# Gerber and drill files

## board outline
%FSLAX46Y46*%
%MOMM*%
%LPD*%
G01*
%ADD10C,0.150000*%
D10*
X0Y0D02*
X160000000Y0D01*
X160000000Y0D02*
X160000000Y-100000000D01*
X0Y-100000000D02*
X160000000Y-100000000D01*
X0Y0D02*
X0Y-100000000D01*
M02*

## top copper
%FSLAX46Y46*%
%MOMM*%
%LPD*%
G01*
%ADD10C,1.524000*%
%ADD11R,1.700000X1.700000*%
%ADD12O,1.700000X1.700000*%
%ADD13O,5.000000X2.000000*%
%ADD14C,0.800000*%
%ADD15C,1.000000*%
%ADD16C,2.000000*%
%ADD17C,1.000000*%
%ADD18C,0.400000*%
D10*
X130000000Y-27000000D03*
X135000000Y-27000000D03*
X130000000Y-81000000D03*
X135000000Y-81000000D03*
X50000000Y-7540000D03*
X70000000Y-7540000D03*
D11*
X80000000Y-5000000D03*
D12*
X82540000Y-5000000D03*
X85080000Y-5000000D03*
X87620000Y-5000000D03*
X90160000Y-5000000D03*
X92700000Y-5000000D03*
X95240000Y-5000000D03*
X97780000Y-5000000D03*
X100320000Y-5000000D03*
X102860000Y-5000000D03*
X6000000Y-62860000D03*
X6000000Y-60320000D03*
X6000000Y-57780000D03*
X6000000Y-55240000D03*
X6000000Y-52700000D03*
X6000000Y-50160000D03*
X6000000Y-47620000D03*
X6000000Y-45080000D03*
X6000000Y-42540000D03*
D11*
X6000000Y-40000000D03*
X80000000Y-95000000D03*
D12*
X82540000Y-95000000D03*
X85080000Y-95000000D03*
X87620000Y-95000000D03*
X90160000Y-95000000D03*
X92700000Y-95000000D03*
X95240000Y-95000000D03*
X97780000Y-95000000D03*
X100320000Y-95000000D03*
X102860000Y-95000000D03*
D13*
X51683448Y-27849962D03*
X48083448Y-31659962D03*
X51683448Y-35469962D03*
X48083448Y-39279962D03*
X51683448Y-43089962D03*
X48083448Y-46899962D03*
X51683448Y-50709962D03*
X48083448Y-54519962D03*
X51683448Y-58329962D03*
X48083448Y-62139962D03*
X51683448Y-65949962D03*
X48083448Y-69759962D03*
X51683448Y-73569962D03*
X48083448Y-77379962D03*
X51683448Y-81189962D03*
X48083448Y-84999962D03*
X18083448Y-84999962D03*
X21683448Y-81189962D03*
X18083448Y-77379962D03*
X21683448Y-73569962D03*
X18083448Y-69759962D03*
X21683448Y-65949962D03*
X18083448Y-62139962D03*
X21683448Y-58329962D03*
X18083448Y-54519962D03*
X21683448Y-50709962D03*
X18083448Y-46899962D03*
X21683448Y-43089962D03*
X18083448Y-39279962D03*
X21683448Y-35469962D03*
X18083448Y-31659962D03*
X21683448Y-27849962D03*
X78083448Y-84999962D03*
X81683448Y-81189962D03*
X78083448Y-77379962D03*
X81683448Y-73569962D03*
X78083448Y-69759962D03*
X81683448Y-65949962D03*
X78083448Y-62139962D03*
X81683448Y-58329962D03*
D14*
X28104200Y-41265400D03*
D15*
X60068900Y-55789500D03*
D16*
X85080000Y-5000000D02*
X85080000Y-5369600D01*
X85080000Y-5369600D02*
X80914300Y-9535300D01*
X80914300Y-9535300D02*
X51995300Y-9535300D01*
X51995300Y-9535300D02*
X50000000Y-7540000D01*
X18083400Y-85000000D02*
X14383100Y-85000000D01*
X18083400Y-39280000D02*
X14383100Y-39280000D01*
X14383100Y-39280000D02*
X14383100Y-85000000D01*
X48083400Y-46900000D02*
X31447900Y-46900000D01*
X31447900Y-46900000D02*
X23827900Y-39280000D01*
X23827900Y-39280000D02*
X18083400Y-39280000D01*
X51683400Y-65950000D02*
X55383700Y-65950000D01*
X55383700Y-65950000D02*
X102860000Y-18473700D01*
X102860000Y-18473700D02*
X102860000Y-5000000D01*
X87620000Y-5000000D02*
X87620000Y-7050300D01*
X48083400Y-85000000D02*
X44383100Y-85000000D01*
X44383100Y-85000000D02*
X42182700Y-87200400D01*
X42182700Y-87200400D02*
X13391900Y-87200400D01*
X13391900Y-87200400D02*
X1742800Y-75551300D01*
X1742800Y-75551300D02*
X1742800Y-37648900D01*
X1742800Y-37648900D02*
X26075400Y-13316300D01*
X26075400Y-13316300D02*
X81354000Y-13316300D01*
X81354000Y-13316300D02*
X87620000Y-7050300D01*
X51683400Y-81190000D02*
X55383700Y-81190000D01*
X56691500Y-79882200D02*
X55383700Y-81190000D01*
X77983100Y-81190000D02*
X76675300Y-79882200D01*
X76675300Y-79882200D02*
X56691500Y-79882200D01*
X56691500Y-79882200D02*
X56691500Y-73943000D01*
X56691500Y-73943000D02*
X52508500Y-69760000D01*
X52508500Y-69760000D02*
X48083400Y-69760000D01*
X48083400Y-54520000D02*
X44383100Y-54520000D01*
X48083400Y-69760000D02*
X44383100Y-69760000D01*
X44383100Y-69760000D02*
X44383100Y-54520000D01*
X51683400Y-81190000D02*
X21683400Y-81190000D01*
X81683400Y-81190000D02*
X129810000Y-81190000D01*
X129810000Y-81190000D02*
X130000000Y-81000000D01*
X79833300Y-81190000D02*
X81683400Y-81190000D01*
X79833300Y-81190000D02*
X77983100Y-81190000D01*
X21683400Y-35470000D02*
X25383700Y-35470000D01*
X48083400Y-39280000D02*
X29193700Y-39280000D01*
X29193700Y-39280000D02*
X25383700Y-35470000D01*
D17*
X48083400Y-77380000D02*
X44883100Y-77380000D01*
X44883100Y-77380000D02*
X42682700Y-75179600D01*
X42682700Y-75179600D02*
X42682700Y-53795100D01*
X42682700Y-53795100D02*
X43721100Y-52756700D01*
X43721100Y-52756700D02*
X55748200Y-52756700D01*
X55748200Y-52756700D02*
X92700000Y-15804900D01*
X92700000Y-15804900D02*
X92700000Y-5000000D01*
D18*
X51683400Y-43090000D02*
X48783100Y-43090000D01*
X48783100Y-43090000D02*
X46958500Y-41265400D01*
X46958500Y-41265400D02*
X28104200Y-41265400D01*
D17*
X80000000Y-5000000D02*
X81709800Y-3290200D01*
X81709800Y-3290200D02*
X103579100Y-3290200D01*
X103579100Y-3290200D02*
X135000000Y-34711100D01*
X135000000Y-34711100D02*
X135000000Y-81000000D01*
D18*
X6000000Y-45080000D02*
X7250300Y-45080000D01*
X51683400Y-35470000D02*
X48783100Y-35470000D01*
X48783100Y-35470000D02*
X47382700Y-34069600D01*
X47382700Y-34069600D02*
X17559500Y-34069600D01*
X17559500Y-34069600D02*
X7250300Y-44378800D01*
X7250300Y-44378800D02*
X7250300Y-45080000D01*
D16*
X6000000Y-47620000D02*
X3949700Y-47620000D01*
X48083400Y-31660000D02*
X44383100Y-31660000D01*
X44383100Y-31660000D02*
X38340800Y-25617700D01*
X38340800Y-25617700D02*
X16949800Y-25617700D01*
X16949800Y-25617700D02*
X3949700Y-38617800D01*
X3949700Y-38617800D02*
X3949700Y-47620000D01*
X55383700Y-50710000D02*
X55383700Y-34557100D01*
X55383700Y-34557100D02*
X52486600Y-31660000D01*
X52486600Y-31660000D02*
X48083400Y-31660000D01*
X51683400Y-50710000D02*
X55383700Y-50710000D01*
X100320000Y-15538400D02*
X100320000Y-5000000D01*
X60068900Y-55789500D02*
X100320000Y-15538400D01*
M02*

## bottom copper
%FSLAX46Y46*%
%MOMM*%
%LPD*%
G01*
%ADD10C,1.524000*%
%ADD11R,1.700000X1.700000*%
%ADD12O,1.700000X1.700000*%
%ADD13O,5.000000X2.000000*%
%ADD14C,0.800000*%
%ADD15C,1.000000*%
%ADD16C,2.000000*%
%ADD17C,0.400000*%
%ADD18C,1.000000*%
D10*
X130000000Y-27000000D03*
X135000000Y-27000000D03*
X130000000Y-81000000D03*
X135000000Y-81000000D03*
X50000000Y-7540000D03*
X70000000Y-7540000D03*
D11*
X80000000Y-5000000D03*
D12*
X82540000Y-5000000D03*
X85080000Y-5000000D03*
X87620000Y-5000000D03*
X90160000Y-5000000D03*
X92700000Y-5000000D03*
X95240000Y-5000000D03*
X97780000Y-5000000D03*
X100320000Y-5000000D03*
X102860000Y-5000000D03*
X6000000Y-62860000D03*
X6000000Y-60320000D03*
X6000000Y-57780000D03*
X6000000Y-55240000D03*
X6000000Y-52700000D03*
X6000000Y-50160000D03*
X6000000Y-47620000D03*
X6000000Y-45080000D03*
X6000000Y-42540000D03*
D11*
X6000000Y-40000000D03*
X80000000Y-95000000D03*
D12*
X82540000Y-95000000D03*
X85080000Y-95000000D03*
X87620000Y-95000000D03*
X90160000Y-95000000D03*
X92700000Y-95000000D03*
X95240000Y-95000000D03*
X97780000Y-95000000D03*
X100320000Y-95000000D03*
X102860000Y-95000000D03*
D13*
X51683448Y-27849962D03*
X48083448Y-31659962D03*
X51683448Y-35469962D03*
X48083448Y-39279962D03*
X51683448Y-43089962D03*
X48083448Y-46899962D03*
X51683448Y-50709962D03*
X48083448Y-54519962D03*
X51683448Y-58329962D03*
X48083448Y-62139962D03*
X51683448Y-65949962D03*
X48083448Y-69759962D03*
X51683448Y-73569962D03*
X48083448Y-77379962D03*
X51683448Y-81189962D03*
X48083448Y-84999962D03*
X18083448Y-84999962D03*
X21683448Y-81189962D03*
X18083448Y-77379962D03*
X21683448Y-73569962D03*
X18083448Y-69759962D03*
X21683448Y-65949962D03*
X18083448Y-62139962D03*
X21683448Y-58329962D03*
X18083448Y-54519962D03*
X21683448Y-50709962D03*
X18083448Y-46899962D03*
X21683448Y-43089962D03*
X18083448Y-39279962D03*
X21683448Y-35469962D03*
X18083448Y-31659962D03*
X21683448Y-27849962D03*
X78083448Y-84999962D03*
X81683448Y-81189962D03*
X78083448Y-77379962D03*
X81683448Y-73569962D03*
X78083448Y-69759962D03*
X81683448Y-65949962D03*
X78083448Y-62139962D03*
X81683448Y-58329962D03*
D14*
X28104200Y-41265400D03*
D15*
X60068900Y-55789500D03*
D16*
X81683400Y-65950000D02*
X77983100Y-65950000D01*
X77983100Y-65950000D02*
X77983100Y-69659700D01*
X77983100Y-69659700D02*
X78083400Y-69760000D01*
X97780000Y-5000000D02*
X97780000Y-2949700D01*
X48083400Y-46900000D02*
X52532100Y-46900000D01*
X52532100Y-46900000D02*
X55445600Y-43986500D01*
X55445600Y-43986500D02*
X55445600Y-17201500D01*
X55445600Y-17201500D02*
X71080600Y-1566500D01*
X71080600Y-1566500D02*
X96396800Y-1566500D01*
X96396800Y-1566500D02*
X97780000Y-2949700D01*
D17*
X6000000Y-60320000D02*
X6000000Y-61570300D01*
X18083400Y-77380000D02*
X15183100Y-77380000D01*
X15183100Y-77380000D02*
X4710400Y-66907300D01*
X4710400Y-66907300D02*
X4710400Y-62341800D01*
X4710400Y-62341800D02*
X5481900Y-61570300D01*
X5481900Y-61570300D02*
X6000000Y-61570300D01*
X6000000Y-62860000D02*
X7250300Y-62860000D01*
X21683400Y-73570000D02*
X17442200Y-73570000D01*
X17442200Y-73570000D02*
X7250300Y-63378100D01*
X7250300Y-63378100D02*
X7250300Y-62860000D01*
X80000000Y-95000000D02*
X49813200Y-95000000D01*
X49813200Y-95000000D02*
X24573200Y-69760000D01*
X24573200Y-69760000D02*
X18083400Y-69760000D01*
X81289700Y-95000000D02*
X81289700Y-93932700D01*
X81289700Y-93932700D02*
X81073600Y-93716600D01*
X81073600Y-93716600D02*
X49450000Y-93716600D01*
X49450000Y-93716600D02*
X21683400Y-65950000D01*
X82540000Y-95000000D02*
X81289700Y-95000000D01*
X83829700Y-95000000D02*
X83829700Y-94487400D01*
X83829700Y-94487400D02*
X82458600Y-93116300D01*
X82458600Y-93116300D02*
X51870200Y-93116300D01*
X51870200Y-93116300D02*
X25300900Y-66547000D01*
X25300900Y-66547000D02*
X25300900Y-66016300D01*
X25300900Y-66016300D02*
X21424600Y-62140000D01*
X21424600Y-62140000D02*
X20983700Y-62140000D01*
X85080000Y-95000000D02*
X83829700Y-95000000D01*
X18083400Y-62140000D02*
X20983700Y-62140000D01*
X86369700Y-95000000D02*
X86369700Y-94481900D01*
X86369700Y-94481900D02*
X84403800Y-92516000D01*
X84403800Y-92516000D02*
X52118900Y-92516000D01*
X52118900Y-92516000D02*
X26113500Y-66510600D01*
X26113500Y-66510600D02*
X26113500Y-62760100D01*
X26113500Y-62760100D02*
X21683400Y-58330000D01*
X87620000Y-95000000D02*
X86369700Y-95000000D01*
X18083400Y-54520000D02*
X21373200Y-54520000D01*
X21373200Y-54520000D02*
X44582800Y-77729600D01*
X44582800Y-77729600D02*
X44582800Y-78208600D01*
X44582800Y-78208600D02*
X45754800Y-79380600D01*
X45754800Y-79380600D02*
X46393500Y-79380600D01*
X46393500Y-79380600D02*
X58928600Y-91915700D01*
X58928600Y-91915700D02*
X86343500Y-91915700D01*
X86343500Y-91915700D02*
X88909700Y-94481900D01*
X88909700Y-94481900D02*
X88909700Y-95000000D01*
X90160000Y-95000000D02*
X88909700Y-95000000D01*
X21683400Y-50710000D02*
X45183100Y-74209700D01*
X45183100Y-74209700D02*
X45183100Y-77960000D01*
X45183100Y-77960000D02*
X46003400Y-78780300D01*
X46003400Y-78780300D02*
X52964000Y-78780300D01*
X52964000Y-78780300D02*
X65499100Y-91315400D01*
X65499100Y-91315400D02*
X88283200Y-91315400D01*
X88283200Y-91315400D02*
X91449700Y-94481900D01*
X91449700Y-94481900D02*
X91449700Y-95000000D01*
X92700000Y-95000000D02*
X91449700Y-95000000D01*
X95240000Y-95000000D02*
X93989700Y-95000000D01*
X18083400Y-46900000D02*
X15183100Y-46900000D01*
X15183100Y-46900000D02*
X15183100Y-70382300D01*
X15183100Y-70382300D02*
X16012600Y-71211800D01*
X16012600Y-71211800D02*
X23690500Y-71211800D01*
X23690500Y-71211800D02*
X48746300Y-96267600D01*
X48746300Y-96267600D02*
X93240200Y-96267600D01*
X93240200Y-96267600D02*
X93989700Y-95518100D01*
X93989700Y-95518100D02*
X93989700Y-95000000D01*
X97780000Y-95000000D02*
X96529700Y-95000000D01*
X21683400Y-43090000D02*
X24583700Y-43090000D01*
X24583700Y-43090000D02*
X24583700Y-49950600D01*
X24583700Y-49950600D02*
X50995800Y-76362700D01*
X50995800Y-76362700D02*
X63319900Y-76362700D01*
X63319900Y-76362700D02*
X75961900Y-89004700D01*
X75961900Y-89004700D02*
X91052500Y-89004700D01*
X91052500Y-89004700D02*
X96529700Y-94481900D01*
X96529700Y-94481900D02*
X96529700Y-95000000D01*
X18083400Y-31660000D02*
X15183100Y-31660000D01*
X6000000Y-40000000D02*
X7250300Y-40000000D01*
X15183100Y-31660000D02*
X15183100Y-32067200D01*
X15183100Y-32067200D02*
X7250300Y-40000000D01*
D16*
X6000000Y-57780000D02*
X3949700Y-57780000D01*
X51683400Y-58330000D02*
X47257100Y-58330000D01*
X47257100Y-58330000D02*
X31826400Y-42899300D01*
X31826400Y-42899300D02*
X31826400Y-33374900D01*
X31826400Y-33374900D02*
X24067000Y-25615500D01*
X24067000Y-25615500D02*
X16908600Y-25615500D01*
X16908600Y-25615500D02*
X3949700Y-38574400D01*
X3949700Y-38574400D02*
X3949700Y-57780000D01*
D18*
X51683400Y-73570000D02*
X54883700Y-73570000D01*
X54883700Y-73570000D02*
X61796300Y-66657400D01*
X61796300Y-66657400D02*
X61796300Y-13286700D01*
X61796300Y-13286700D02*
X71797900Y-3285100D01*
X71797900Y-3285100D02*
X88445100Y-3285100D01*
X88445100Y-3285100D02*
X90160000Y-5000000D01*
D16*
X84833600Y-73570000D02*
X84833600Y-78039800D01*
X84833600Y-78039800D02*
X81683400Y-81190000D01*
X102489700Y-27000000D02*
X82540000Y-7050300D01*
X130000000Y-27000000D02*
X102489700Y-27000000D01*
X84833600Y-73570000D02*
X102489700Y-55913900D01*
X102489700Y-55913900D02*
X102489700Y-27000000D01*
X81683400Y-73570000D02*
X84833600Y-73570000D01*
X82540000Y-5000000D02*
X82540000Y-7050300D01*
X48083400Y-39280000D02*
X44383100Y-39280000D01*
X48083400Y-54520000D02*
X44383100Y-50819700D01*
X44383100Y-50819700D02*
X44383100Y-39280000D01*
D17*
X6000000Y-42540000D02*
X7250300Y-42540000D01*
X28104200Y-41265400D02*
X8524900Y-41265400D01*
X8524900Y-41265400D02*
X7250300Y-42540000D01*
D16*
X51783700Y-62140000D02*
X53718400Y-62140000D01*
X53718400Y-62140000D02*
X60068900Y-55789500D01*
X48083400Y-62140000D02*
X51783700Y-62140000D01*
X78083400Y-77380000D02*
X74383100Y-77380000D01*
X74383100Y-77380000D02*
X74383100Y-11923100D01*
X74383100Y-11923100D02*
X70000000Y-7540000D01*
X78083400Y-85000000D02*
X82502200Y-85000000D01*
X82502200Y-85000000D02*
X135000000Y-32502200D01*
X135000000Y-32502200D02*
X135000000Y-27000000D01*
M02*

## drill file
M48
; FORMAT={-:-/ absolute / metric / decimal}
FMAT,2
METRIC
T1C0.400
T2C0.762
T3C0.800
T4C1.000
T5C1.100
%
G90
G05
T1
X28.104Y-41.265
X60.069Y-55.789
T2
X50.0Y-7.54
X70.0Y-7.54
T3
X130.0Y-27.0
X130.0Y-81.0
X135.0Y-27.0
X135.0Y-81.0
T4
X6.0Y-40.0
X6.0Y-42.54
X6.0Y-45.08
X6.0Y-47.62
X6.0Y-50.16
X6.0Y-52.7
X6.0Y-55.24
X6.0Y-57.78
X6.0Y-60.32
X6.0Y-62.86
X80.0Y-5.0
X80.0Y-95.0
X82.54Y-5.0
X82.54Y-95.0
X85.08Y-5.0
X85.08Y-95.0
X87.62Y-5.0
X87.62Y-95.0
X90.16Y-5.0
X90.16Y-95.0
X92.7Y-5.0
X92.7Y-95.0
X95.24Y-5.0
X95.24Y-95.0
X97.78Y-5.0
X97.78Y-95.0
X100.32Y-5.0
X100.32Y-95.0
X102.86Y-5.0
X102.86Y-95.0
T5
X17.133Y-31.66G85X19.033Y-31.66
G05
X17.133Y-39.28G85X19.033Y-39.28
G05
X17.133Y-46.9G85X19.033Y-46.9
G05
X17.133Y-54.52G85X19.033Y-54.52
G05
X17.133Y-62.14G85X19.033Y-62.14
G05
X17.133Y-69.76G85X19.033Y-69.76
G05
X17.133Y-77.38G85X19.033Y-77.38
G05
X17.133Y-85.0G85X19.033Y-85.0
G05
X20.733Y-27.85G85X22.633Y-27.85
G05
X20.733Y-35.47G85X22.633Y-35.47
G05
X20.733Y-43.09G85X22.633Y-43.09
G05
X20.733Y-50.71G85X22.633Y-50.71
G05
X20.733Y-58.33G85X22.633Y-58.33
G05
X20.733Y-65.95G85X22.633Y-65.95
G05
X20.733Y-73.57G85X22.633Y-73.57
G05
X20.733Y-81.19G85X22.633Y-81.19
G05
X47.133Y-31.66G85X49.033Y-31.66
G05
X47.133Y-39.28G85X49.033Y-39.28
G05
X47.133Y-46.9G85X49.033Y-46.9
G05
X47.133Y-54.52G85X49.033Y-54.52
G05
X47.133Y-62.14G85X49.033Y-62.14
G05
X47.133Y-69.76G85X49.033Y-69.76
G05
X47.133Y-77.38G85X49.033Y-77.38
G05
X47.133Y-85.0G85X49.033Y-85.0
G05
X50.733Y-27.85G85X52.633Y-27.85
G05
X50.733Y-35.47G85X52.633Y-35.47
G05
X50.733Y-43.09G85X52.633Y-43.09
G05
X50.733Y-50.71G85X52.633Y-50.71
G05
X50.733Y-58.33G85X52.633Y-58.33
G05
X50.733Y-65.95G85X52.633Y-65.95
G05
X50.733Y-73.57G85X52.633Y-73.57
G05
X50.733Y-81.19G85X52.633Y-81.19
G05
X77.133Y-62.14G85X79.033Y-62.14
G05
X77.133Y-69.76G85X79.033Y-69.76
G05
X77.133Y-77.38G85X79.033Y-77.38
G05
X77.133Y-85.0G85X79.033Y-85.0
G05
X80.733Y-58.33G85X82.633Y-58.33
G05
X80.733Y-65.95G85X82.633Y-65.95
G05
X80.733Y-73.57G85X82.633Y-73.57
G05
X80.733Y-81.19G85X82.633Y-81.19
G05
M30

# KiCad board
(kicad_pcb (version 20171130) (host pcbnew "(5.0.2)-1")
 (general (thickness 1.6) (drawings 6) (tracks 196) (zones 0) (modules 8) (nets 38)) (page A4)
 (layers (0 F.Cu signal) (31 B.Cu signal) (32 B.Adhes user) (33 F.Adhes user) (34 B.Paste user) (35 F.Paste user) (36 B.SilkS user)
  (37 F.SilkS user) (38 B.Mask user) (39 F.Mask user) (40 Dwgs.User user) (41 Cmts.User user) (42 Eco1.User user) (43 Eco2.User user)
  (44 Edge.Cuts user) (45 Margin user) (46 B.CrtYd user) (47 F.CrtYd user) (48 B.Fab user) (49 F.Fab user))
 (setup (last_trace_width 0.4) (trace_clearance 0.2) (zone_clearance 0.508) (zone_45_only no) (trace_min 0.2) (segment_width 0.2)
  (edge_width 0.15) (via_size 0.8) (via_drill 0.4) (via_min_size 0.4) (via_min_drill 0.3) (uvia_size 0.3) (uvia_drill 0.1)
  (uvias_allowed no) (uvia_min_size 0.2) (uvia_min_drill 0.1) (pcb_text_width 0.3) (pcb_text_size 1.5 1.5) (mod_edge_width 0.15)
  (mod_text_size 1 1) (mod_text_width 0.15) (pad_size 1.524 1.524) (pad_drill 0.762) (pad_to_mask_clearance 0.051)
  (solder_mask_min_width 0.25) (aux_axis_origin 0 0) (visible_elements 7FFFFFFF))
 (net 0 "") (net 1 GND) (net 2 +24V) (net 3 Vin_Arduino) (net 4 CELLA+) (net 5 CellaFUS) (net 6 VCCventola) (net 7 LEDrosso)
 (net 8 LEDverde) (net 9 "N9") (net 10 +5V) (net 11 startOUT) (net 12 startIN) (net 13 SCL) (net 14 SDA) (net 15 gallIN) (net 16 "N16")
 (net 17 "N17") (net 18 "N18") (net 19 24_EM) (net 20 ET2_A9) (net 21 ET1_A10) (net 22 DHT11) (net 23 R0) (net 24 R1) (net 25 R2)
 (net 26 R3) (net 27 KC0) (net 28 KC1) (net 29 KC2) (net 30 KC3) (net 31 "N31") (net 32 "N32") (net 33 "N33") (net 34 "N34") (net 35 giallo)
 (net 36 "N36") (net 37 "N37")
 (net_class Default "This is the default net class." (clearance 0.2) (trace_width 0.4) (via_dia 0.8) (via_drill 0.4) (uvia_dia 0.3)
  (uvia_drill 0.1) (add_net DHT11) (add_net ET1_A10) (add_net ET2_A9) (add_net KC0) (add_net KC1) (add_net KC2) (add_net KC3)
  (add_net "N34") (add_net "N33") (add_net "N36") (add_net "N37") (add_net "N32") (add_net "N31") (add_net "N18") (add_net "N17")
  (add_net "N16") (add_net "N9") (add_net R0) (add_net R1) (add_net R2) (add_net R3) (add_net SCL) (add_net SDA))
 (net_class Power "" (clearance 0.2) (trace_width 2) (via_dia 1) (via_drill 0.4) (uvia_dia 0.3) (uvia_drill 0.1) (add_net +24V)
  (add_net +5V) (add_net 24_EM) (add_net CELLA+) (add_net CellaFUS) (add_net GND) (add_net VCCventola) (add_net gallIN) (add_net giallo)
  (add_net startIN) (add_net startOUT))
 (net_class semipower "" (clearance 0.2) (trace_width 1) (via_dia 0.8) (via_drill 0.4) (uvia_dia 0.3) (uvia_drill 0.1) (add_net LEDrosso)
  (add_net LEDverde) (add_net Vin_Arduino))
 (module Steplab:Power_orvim (layer F.Cu) (at 130 23)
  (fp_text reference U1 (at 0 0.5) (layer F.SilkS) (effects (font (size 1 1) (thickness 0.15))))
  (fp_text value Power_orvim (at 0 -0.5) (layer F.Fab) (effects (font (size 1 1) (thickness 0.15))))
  (pad 2 thru_hole circle (at 0 4) (size 1.524 1.524) (drill 0.8) (layers *.Cu *.Mask) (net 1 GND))
  (pad 1 thru_hole circle (at 5 4) (size 1.524 1.524) (drill 0.8) (layers *.Cu *.Mask) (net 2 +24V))
  (pad 4 thru_hole circle (at 0 58) (size 1.524 1.524) (drill 0.8) (layers *.Cu *.Mask) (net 1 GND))
  (pad 3 thru_hole circle (at 5 58) (size 1.524 1.524) (drill 0.8) (layers *.Cu *.Mask) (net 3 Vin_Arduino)))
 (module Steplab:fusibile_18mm (layer F.Cu) (at 51.95 5)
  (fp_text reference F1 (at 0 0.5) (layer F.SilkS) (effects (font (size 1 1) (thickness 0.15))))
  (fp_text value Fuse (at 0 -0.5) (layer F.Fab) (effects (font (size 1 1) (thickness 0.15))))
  (pad 1 thru_hole circle (at -1.95 2.54) (size 1.524 1.524) (drill 0.762) (layers *.Cu *.Mask) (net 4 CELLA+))
  (pad 2 thru_hole circle (at 18.05 2.54) (size 1.524 1.524) (drill 0.762) (layers *.Cu *.Mask) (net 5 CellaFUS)))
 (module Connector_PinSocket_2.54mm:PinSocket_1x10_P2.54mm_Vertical (layer F.Cu) (at 80 5 90)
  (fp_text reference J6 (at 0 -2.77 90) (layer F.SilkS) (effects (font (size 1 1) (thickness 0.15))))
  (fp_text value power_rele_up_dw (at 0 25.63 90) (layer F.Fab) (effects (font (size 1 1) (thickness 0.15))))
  (pad 1 thru_hole rect (at 0 0 90) (size 1.7 1.7) (drill 1) (layers *.Cu *.Mask) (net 3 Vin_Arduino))
  (pad 2 thru_hole oval (at 0 2.54 90) (size 1.7 1.7) (drill 1) (layers *.Cu *.Mask) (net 1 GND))
  (pad 3 thru_hole oval (at 0 5.08 90) (size 1.7 1.7) (drill 1) (layers *.Cu *.Mask) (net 4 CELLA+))
  (pad 4 thru_hole oval (at 0 7.62 90) (size 1.7 1.7) (drill 1) (layers *.Cu *.Mask) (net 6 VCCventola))
  (pad 5 thru_hole oval (at 0 10.16 90) (size 1.7 1.7) (drill 1) (layers *.Cu *.Mask) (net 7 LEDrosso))
  (pad 6 thru_hole oval (at 0 12.7 90) (size 1.7 1.7) (drill 1) (layers *.Cu *.Mask) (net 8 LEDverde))
  (pad 7 thru_hole oval (at 0 15.24 90) (size 1.7 1.7) (drill 1) (layers *.Cu *.Mask) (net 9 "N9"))
  (pad 8 thru_hole oval (at 0 17.78 90) (size 1.7 1.7) (drill 1) (layers *.Cu *.Mask) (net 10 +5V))
  (pad 9 thru_hole oval (at 0 20.32 90) (size 1.7 1.7) (drill 1) (layers *.Cu *.Mask) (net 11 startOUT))
  (pad 10 thru_hole oval (at 0 22.86 90) (size 1.7 1.7) (drill 1) (layers *.Cu *.Mask) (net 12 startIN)))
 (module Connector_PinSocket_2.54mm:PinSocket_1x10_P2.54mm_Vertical (layer F.Cu) (at 6 40)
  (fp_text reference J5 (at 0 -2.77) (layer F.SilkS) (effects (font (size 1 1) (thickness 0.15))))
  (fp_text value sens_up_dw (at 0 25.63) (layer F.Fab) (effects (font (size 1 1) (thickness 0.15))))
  (pad 10 thru_hole oval (at 0 22.86) (size 1.7 1.7) (drill 1) (layers *.Cu *.Mask) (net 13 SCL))
  (pad 9 thru_hole oval (at 0 20.32) (size 1.7 1.7) (drill 1) (layers *.Cu *.Mask) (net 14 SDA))
  (pad 8 thru_hole oval (at 0 17.78) (size 1.7 1.7) (drill 1) (layers *.Cu *.Mask) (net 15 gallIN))
  (pad 7 thru_hole oval (at 0 15.24) (size 1.7 1.7) (drill 1) (layers *.Cu *.Mask) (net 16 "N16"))
  (pad 6 thru_hole oval (at 0 12.7) (size 1.7 1.7) (drill 1) (layers *.Cu *.Mask) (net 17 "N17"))
  (pad 5 thru_hole oval (at 0 10.16) (size 1.7 1.7) (drill 1) (layers *.Cu *.Mask) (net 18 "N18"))
  (pad 4 thru_hole oval (at 0 7.62) (size 1.7 1.7) (drill 1) (layers *.Cu *.Mask) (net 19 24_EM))
  (pad 3 thru_hole oval (at 0 5.08) (size 1.7 1.7) (drill 1) (layers *.Cu *.Mask) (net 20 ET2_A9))
  (pad 2 thru_hole oval (at 0 2.54) (size 1.7 1.7) (drill 1) (layers *.Cu *.Mask) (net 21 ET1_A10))
  (pad 1 thru_hole rect (at 0 0) (size 1.7 1.7) (drill 1) (layers *.Cu *.Mask) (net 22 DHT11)))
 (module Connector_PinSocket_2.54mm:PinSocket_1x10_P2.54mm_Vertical (layer F.Cu) (at 80 95 90)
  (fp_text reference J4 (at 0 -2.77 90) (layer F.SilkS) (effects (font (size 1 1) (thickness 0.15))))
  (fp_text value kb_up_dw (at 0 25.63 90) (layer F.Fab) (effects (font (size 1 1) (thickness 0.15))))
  (pad 1 thru_hole rect (at 0 0 90) (size 1.7 1.7) (drill 1) (layers *.Cu *.Mask) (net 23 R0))
  (pad 2 thru_hole oval (at 0 2.54 90) (size 1.7 1.7) (drill 1) (layers *.Cu *.Mask) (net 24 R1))
  (pad 3 thru_hole oval (at 0 5.08 90) (size 1.7 1.7) (drill 1) (layers *.Cu *.Mask) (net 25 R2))
  (pad 4 thru_hole oval (at 0 7.62 90) (size 1.7 1.7) (drill 1) (layers *.Cu *.Mask) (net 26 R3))
  (pad 5 thru_hole oval (at 0 10.16 90) (size 1.7 1.7) (drill 1) (layers *.Cu *.Mask) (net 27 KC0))
  (pad 6 thru_hole oval (at 0 12.7 90) (size 1.7 1.7) (drill 1) (layers *.Cu *.Mask) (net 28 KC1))
  (pad 7 thru_hole oval (at 0 15.24 90) (size 1.7 1.7) (drill 1) (layers *.Cu *.Mask) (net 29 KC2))
  (pad 8 thru_hole oval (at 0 17.78 90) (size 1.7 1.7) (drill 1) (layers *.Cu *.Mask) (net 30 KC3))
  (pad 9 thru_hole oval (at 0 20.32 90) (size 1.7 1.7) (drill 1) (layers *.Cu *.Mask) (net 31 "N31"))
  (pad 10 thru_hole oval (at 0 22.86 90) (size 1.7 1.7) (drill 1) (layers *.Cu *.Mask) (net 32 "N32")))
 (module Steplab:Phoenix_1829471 (layer F.Cu) (at 52 68.5137 180)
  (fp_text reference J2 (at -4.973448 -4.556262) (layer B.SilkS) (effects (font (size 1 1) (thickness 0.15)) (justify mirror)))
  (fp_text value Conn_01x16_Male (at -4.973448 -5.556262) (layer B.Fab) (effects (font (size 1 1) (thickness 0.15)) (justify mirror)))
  (pad 16 thru_hole oval (at 0.316552 40.663738) (size 5 2) (drill oval 3 1.1) (layers *.Cu *.Mask) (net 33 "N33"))
  (pad 15 thru_hole oval (at 3.916552 36.853738) (size 5 2) (drill oval 3 1.1) (layers *.Cu *.Mask) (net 19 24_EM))
  (pad 14 thru_hole oval (at 0.316552 33.043738) (size 5 2) (drill oval 3 1.1) (layers *.Cu *.Mask) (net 20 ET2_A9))
  (pad 13 thru_hole oval (at 3.916552 29.233738) (size 5 2) (drill oval 3 1.1) (layers *.Cu *.Mask) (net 1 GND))
  (pad 12 thru_hole oval (at 0.316552 25.423738) (size 5 2) (drill oval 3 1.1) (layers *.Cu *.Mask) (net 21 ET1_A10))
  (pad 11 thru_hole oval (at 3.916552 21.613738) (size 5 2) (drill oval 3 1.1) (layers *.Cu *.Mask) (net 10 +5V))
  (pad 10 thru_hole oval (at 0.316552 17.803738) (size 5 2) (drill oval 3 1.1) (layers *.Cu *.Mask) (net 19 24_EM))
  (pad 9 thru_hole oval (at 3.916552 13.993738) (size 5 2) (drill oval 3 1.1) (layers *.Cu *.Mask) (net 1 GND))
  (pad 8 thru_hole oval (at 0.316552 10.183738) (size 5 2) (drill oval 3 1.1) (layers *.Cu *.Mask) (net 15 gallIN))
  (pad 7 thru_hole oval (at 3.916552 6.373738) (size 5 2) (drill oval 3 1.1) (layers *.Cu *.Mask) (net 11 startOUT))
  (pad 6 thru_hole oval (at 0.316552 2.563738) (size 5 2) (drill oval 3 1.1) (layers *.Cu *.Mask) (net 12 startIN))
  (pad 5 thru_hole oval (at 3.916552 -1.246262) (size 5 2) (drill oval 3 1.1) (layers *.Cu *.Mask) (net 1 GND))
  (pad 4 thru_hole oval (at 0.316552 -5.056262) (size 5 2) (drill oval 3 1.1) (layers *.Cu *.Mask) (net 7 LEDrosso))
  (pad 3 thru_hole oval (at 3.916552 -8.866262) (size 5 2) (drill oval 3 1.1) (layers *.Cu *.Mask) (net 8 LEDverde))
  (pad 2 thru_hole oval (at 0.316552 -12.676262) (size 5 2) (drill oval 3 1.1) (layers *.Cu *.Mask) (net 1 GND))
  (pad 1 thru_hole oval (at 3.916552 -16.486262) (size 5 2) (drill oval 3 1.1) (layers *.Cu *.Mask) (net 6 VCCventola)))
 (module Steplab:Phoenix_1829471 (layer F.Cu) (at 22 68.5137 180)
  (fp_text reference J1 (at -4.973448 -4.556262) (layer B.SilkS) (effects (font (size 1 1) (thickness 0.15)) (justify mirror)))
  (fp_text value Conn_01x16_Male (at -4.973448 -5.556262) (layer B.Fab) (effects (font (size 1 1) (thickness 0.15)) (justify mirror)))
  (pad 1 thru_hole oval (at 3.916552 -16.486262) (size 5 2) (drill oval 3 1.1) (layers *.Cu *.Mask) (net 10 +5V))
  (pad 2 thru_hole oval (at 0.316552 -12.676262) (size 5 2) (drill oval 3 1.1) (layers *.Cu *.Mask) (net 1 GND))
  (pad 3 thru_hole oval (at 3.916552 -8.866262) (size 5 2) (drill oval 3 1.1) (layers *.Cu *.Mask) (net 14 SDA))
  (pad 4 thru_hole oval (at 0.316552 -5.056262) (size 5 2) (drill oval 3 1.1) (layers *.Cu *.Mask) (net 13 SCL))
  (pad 5 thru_hole oval (at 3.916552 -1.246262) (size 5 2) (drill oval 3 1.1) (layers *.Cu *.Mask) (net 23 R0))
  (pad 6 thru_hole oval (at 0.316552 2.563738) (size 5 2) (drill oval 3 1.1) (layers *.Cu *.Mask) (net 24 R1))
  (pad 7 thru_hole oval (at 3.916552 6.373738) (size 5 2) (drill oval 3 1.1) (layers *.Cu *.Mask) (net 25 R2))
  (pad 8 thru_hole oval (at 0.316552 10.183738) (size 5 2) (drill oval 3 1.1) (layers *.Cu *.Mask) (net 26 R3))
  (pad 9 thru_hole oval (at 3.916552 13.993738) (size 5 2) (drill oval 3 1.1) (layers *.Cu *.Mask) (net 27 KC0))
  (pad 10 thru_hole oval (at 0.316552 17.803738) (size 5 2) (drill oval 3 1.1) (layers *.Cu *.Mask) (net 28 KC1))
  (pad 11 thru_hole oval (at 3.916552 21.613738) (size 5 2) (drill oval 3 1.1) (layers *.Cu *.Mask) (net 29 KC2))
  (pad 12 thru_hole oval (at 0.316552 25.423738) (size 5 2) (drill oval 3 1.1) (layers *.Cu *.Mask) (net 30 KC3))
  (pad 13 thru_hole oval (at 3.916552 29.233738) (size 5 2) (drill oval 3 1.1) (layers *.Cu *.Mask) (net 10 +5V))
  (pad 14 thru_hole oval (at 0.316552 33.043738) (size 5 2) (drill oval 3 1.1) (layers *.Cu *.Mask) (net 1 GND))
  (pad 15 thru_hole oval (at 3.916552 36.853738) (size 5 2) (drill oval 3 1.1) (layers *.Cu *.Mask) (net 22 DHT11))
  (pad 16 thru_hole oval (at 0.316552 40.663738) (size 5 2) (drill oval 3 1.1) (layers *.Cu *.Mask) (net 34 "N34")))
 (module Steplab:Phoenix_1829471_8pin (layer F.Cu) (at 82 68.5137 180)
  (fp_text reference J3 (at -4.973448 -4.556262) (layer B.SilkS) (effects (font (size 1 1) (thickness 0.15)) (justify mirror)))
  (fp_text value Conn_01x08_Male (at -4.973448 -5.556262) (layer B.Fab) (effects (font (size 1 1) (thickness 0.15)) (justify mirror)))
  (pad 1 thru_hole oval (at 3.916552 -16.486262) (size 5 2) (drill oval 3 1.1) (layers *.Cu *.Mask) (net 2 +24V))
  (pad 2 thru_hole oval (at 0.316552 -12.676262) (size 5 2) (drill oval 3 1.1) (layers *.Cu *.Mask) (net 1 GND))
  (pad 3 thru_hole oval (at 3.916552 -8.866262) (size 5 2) (drill oval 3 1.1) (layers *.Cu *.Mask) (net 5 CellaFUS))
  (pad 4 thru_hole oval (at 0.316552 -5.056262) (size 5 2) (drill oval 3 1.1) (layers *.Cu *.Mask) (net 1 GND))
  (pad 5 thru_hole oval (at 3.916552 -1.246262) (size 5 2) (drill oval 3 1.1) (layers *.Cu *.Mask) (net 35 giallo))
  (pad 6 thru_hole oval (at 0.316552 2.563738) (size 5 2) (drill oval 3 1.1) (layers *.Cu *.Mask) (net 35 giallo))
  (pad 7 thru_hole oval (at 3.916552 6.373738) (size 5 2) (drill oval 3 1.1) (layers *.Cu *.Mask) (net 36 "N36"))
  (pad 8 thru_hole oval (at 0.316552 10.183738) (size 5 2) (drill oval 3 1.1) (layers *.Cu *.Mask) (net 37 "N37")))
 (gr_line (start 0 0) (end 160 0) (layer Edge.Cuts) (width 0.15))
 (gr_line (start 160 0) (end 160 100) (layer Edge.Cuts) (width 0.15))
 (gr_line (start 0 100) (end 160 100) (layer Edge.Cuts) (width 0.15))
 (gr_line (start 0 0) (end 0 100) (layer Edge.Cuts) (width 0.15))
 (segment (start 85.08 5) (end 85.08 5.3696) (width 2) (layer F.Cu) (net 4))
 (segment (start 85.08 5.3696) (end 80.9143 9.5353) (width 2) (layer F.Cu) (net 4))
 (segment (start 80.9143 9.5353) (end 51.9953 9.5353) (width 2) (layer F.Cu) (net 4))
 (segment (start 51.9953 9.5353) (end 50 7.54) (width 2) (layer F.Cu) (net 4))
 (segment (start 81.6834 65.95) (end 77.9831 65.95) (width 2) (layer B.Cu) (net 35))
 (segment (start 77.9831 65.95) (end 77.9831 69.6597) (width 2) (layer B.Cu) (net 35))
 (segment (start 77.9831 69.6597) (end 78.0834 69.76) (width 2) (layer B.Cu) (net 35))
 (segment (start 18.0834 85) (end 14.3831 85) (width 2) (layer F.Cu) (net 10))
 (segment (start 18.0834 39.28) (end 14.3831 39.28) (width 2) (layer F.Cu) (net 10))
 (segment (start 14.3831 39.28) (end 14.3831 85) (width 2) (layer F.Cu) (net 10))
 (segment (start 48.0834 46.9) (end 31.4479 46.9) (width 2) (layer F.Cu) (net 10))
 (segment (start 31.4479 46.9) (end 23.8279 39.28) (width 2) (layer F.Cu) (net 10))
 (segment (start 23.8279 39.28) (end 18.0834 39.28) (width 2) (layer F.Cu) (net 10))
 (segment (start 97.78 5) (end 97.78 2.9497) (width 2) (layer B.Cu) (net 10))
 (segment (start 48.0834 46.9) (end 52.5321 46.9) (width 2) (layer B.Cu) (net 10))
 (segment (start 52.5321 46.9) (end 55.4456 43.9865) (width 2) (layer B.Cu) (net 10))
 (segment (start 55.4456 43.9865) (end 55.4456 17.2015) (width 2) (layer B.Cu) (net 10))
 (segment (start 55.4456 17.2015) (end 71.0806 1.5665) (width 2) (layer B.Cu) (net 10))
 (segment (start 71.0806 1.5665) (end 96.3968 1.5665) (width 2) (layer B.Cu) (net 10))
 (segment (start 96.3968 1.5665) (end 97.78 2.9497) (width 2) (layer B.Cu) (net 10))
 (segment (start 6 60.32) (end 6 61.5703) (width 0.4) (layer B.Cu) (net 14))
 (segment (start 18.0834 77.38) (end 15.1831 77.38) (width 0.4) (layer B.Cu) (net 14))
 (segment (start 15.1831 77.38) (end 4.7104 66.9073) (width 0.4) (layer B.Cu) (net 14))
 (segment (start 4.7104 66.9073) (end 4.7104 62.3418) (width 0.4) (layer B.Cu) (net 14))
 (segment (start 4.7104 62.3418) (end 5.4819 61.5703) (width 0.4) (layer B.Cu) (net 14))
 (segment (start 5.4819 61.5703) (end 6 61.5703) (width 0.4) (layer B.Cu) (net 14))
 (segment (start 6 62.86) (end 7.2503 62.86) (width 0.4) (layer B.Cu) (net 13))
 (segment (start 21.6834 73.57) (end 17.4422 73.57) (width 0.4) (layer B.Cu) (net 13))
 (segment (start 17.4422 73.57) (end 7.2503 63.3781) (width 0.4) (layer B.Cu) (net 13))
 (segment (start 7.2503 63.3781) (end 7.2503 62.86) (width 0.4) (layer B.Cu) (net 13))
 (segment (start 80 95) (end 49.8132 95) (width 0.4) (layer B.Cu) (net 23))
 (segment (start 49.8132 95) (end 24.5732 69.76) (width 0.4) (layer B.Cu) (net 23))
 (segment (start 24.5732 69.76) (end 18.0834 69.76) (width 0.4) (layer B.Cu) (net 23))
 (segment (start 81.2897 95) (end 81.2897 93.9327) (width 0.4) (layer B.Cu) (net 24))
 (segment (start 81.2897 93.9327) (end 81.0736 93.7166) (width 0.4) (layer B.Cu) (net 24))
 (segment (start 81.0736 93.7166) (end 49.45 93.7166) (width 0.4) (layer B.Cu) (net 24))
 (segment (start 49.45 93.7166) (end 21.6834 65.95) (width 0.4) (layer B.Cu) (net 24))
 (segment (start 82.54 95) (end 81.2897 95) (width 0.4) (layer B.Cu) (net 24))
 (segment (start 83.8297 95) (end 83.8297 94.4874) (width 0.4) (layer B.Cu) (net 25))
 (segment (start 83.8297 94.4874) (end 82.4586 93.1163) (width 0.4) (layer B.Cu) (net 25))
 (segment (start 82.4586 93.1163) (end 51.8702 93.1163) (width 0.4) (layer B.Cu) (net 25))
 (segment (start 51.8702 93.1163) (end 25.3009 66.547) (width 0.4) (layer B.Cu) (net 25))
 (segment (start 25.3009 66.547) (end 25.3009 66.0163) (width 0.4) (layer B.Cu) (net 25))
 (segment (start 25.3009 66.0163) (end 21.4246 62.14) (width 0.4) (layer B.Cu) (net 25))
 (segment (start 21.4246 62.14) (end 20.9837 62.14) (width 0.4) (layer B.Cu) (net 25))
 (segment (start 85.08 95) (end 83.8297 95) (width 0.4) (layer B.Cu) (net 25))
 (segment (start 18.0834 62.14) (end 20.9837 62.14) (width 0.4) (layer B.Cu) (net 25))
 (segment (start 86.3697 95) (end 86.3697 94.4819) (width 0.4) (layer B.Cu) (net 26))
 (segment (start 86.3697 94.4819) (end 84.4038 92.516) (width 0.4) (layer B.Cu) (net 26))
 (segment (start 84.4038 92.516) (end 52.1189 92.516) (width 0.4) (layer B.Cu) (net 26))
 (segment (start 52.1189 92.516) (end 26.1135 66.5106) (width 0.4) (layer B.Cu) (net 26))
 (segment (start 26.1135 66.5106) (end 26.1135 62.7601) (width 0.4) (layer B.Cu) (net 26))
 (segment (start 26.1135 62.7601) (end 21.6834 58.33) (width 0.4) (layer B.Cu) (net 26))
 (segment (start 87.62 95) (end 86.3697 95) (width 0.4) (layer B.Cu) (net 26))
 (segment (start 18.0834 54.52) (end 21.3732 54.52) (width 0.4) (layer B.Cu) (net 27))
 (segment (start 21.3732 54.52) (end 44.5828 77.7296) (width 0.4) (layer B.Cu) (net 27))
 (segment (start 44.5828 77.7296) (end 44.5828 78.2086) (width 0.4) (layer B.Cu) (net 27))
 (segment (start 44.5828 78.2086) (end 45.7548 79.3806) (width 0.4) (layer B.Cu) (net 27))
 (segment (start 45.7548 79.3806) (end 46.3935 79.3806) (width 0.4) (layer B.Cu) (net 27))
 (segment (start 46.3935 79.3806) (end 58.9286 91.9157) (width 0.4) (layer B.Cu) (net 27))
 (segment (start 58.9286 91.9157) (end 86.3435 91.9157) (width 0.4) (layer B.Cu) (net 27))
 (segment (start 86.3435 91.9157) (end 88.9097 94.4819) (width 0.4) (layer B.Cu) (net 27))
 (segment (start 88.9097 94.4819) (end 88.9097 95) (width 0.4) (layer B.Cu) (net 27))
 (segment (start 90.16 95) (end 88.9097 95) (width 0.4) (layer B.Cu) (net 27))
 (segment (start 21.6834 50.71) (end 45.1831 74.2097) (width 0.4) (layer B.Cu) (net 28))
 (segment (start 45.1831 74.2097) (end 45.1831 77.96) (width 0.4) (layer B.Cu) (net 28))
 (segment (start 45.1831 77.96) (end 46.0034 78.7803) (width 0.4) (layer B.Cu) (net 28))
 (segment (start 46.0034 78.7803) (end 52.964 78.7803) (width 0.4) (layer B.Cu) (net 28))
 (segment (start 52.964 78.7803) (end 65.4991 91.3154) (width 0.4) (layer B.Cu) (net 28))
 (segment (start 65.4991 91.3154) (end 88.2832 91.3154) (width 0.4) (layer B.Cu) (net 28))
 (segment (start 88.2832 91.3154) (end 91.4497 94.4819) (width 0.4) (layer B.Cu) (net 28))
 (segment (start 91.4497 94.4819) (end 91.4497 95) (width 0.4) (layer B.Cu) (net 28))
 (segment (start 92.7 95) (end 91.4497 95) (width 0.4) (layer B.Cu) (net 28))
 (segment (start 95.24 95) (end 93.9897 95) (width 0.4) (layer B.Cu) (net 29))
 (segment (start 18.0834 46.9) (end 15.1831 46.9) (width 0.4) (layer B.Cu) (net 29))
 (segment (start 15.1831 46.9) (end 15.1831 70.3823) (width 0.4) (layer B.Cu) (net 29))
 (segment (start 15.1831 70.3823) (end 16.0126 71.2118) (width 0.4) (layer B.Cu) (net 29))
 (segment (start 16.0126 71.2118) (end 23.6905 71.2118) (width 0.4) (layer B.Cu) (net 29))
 (segment (start 23.6905 71.2118) (end 48.7463 96.2676) (width 0.4) (layer B.Cu) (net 29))
 (segment (start 48.7463 96.2676) (end 93.2402 96.2676) (width 0.4) (layer B.Cu) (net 29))
 (segment (start 93.2402 96.2676) (end 93.9897 95.5181) (width 0.4) (layer B.Cu) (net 29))
 (segment (start 93.9897 95.5181) (end 93.9897 95) (width 0.4) (layer B.Cu) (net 29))
 (segment (start 97.78 95) (end 96.5297 95) (width 0.4) (layer B.Cu) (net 30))
 (segment (start 21.6834 43.09) (end 24.5837 43.09) (width 0.4) (layer B.Cu) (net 30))
 (segment (start 24.5837 43.09) (end 24.5837 49.9506) (width 0.4) (layer B.Cu) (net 30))
 (segment (start 24.5837 49.9506) (end 50.9958 76.3627) (width 0.4) (layer B.Cu) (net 30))
 (segment (start 50.9958 76.3627) (end 63.3199 76.3627) (width 0.4) (layer B.Cu) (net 30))
 (segment (start 63.3199 76.3627) (end 75.9619 89.0047) (width 0.4) (layer B.Cu) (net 30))
 (segment (start 75.9619 89.0047) (end 91.0525 89.0047) (width 0.4) (layer B.Cu) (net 30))
 (segment (start 91.0525 89.0047) (end 96.5297 94.4819) (width 0.4) (layer B.Cu) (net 30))
 (segment (start 96.5297 94.4819) (end 96.5297 95) (width 0.4) (layer B.Cu) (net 30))
 (segment (start 18.0834 31.66) (end 15.1831 31.66) (width 0.4) (layer B.Cu) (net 22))
 (segment (start 6 40) (end 7.2503 40) (width 0.4) (layer B.Cu) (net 22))
 (segment (start 15.1831 31.66) (end 15.1831 32.0672) (width 0.4) (layer B.Cu) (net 22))
 (segment (start 15.1831 32.0672) (end 7.2503 40) (width 0.4) (layer B.Cu) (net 22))
 (segment (start 6 57.78) (end 3.9497 57.78) (width 2) (layer B.Cu) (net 15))
 (segment (start 51.6834 58.33) (end 47.2571 58.33) (width 2) (layer B.Cu) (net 15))
 (segment (start 47.2571 58.33) (end 31.8264 42.8993) (width 2) (layer B.Cu) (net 15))
 (segment (start 31.8264 42.8993) (end 31.8264 33.3749) (width 2) (layer B.Cu) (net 15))
 (segment (start 31.8264 33.3749) (end 24.067 25.6155) (width 2) (layer B.Cu) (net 15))
 (segment (start 24.067 25.6155) (end 16.9086 25.6155) (width 2) (layer B.Cu) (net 15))
 (segment (start 16.9086 25.6155) (end 3.9497 38.5744) (width 2) (layer B.Cu) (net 15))
 (segment (start 3.9497 38.5744) (end 3.9497 57.78) (width 2) (layer B.Cu) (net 15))
 (segment (start 51.6834 65.95) (end 55.3837 65.95) (width 2) (layer F.Cu) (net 12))
 (segment (start 55.3837 65.95) (end 102.86 18.4737) (width 2) (layer F.Cu) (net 12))
 (segment (start 102.86 18.4737) (end 102.86 5) (width 2) (layer F.Cu) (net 12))
 (segment (start 51.6834 73.57) (end 54.8837 73.57) (width 1) (layer B.Cu) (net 7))
 (segment (start 54.8837 73.57) (end 61.7963 66.6574) (width 1) (layer B.Cu) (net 7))
 (segment (start 61.7963 66.6574) (end 61.7963 13.2867) (width 1) (layer B.Cu) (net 7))
 (segment (start 61.7963 13.2867) (end 71.7979 3.2851) (width 1) (layer B.Cu) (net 7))
 (segment (start 71.7979 3.2851) (end 88.4451 3.2851) (width 1) (layer B.Cu) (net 7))
 (segment (start 88.4451 3.2851) (end 90.16 5) (width 1) (layer B.Cu) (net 7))
 (segment (start 87.62 5) (end 87.62 7.0503) (width 2) (layer F.Cu) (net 6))
 (segment (start 48.0834 85) (end 44.3831 85) (width 2) (layer F.Cu) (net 6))
 (segment (start 44.3831 85) (end 42.1827 87.2004) (width 2) (layer F.Cu) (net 6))
 (segment (start 42.1827 87.2004) (end 13.3919 87.2004) (width 2) (layer F.Cu) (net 6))
 (segment (start 13.3919 87.2004) (end 1.7428 75.5513) (width 2) (layer F.Cu) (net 6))
 (segment (start 1.7428 75.5513) (end 1.7428 37.6489) (width 2) (layer F.Cu) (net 6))
 (segment (start 1.7428 37.6489) (end 26.0754 13.3163) (width 2) (layer F.Cu) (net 6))
 (segment (start 26.0754 13.3163) (end 81.354 13.3163) (width 2) (layer F.Cu) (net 6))
 (segment (start 81.354 13.3163) (end 87.62 7.0503) (width 2) (layer F.Cu) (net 6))
 (segment (start 51.6834 81.19) (end 55.3837 81.19) (width 2) (layer F.Cu) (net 1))
 (segment (start 56.6915 79.8822) (end 55.3837 81.19) (width 2) (layer F.Cu) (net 1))
 (segment (start 77.9831 81.19) (end 76.6753 79.8822) (width 2) (layer F.Cu) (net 1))
 (segment (start 76.6753 79.8822) (end 56.6915 79.8822) (width 2) (layer F.Cu) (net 1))
 (segment (start 56.6915 79.8822) (end 56.6915 73.943) (width 2) (layer F.Cu) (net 1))
 (segment (start 56.6915 73.943) (end 52.5085 69.76) (width 2) (layer F.Cu) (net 1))
 (segment (start 52.5085 69.76) (end 48.0834 69.76) (width 2) (layer F.Cu) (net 1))
 (segment (start 48.0834 54.52) (end 44.3831 54.52) (width 2) (layer F.Cu) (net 1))
 (segment (start 48.0834 69.76) (end 44.3831 69.76) (width 2) (layer F.Cu) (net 1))
 (segment (start 44.3831 69.76) (end 44.3831 54.52) (width 2) (layer F.Cu) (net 1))
 (segment (start 51.6834 81.19) (end 21.6834 81.19) (width 2) (layer F.Cu) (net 1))
 (segment (start 84.8336 73.57) (end 84.8336 78.0398) (width 2) (layer B.Cu) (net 1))
 (segment (start 84.8336 78.0398) (end 81.6834 81.19) (width 2) (layer B.Cu) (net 1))
 (segment (start 102.4897 27) (end 82.54 7.0503) (width 2) (layer B.Cu) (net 1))
 (segment (start 130 27) (end 102.4897 27) (width 2) (layer B.Cu) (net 1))
 (segment (start 84.8336 73.57) (end 102.4897 55.9139) (width 2) (layer B.Cu) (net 1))
 (segment (start 102.4897 55.9139) (end 102.4897 27) (width 2) (layer B.Cu) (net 1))
 (segment (start 81.6834 73.57) (end 84.8336 73.57) (width 2) (layer B.Cu) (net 1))
 (segment (start 81.6834 81.19) (end 129.81 81.19) (width 2) (layer F.Cu) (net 1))
 (segment (start 129.81 81.19) (end 130 81) (width 2) (layer F.Cu) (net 1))
 (segment (start 79.8333 81.19) (end 81.6834 81.19) (width 2) (layer F.Cu) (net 1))
 (segment (start 79.8333 81.19) (end 77.9831 81.19) (width 2) (layer F.Cu) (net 1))
 (segment (start 82.54 5) (end 82.54 7.0503) (width 2) (layer B.Cu) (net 1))
 (segment (start 48.0834 39.28) (end 44.3831 39.28) (width 2) (layer B.Cu) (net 1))
 (segment (start 48.0834 54.52) (end 44.3831 50.8197) (width 2) (layer B.Cu) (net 1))
 (segment (start 44.3831 50.8197) (end 44.3831 39.28) (width 2) (layer B.Cu) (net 1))
 (segment (start 21.6834 35.47) (end 25.3837 35.47) (width 2) (layer F.Cu) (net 1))
 (segment (start 48.0834 39.28) (end 29.1937 39.28) (width 2) (layer F.Cu) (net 1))
 (segment (start 29.1937 39.28) (end 25.3837 35.47) (width 2) (layer F.Cu) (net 1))
 (segment (start 48.0834 77.38) (end 44.8831 77.38) (width 1) (layer F.Cu) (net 8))
 (segment (start 44.8831 77.38) (end 42.6827 75.1796) (width 1) (layer F.Cu) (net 8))
 (segment (start 42.6827 75.1796) (end 42.6827 53.7951) (width 1) (layer F.Cu) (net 8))
 (segment (start 42.6827 53.7951) (end 43.7211 52.7567) (width 1) (layer F.Cu) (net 8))
 (segment (start 43.7211 52.7567) (end 55.7482 52.7567) (width 1) (layer F.Cu) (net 8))
 (segment (start 55.7482 52.7567) (end 92.7 15.8049) (width 1) (layer F.Cu) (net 8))
 (segment (start 92.7 15.8049) (end 92.7 5) (width 1) (layer F.Cu) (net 8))
 (segment (start 51.6834 43.09) (end 48.7831 43.09) (width 0.4) (layer F.Cu) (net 21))
 (segment (start 6 42.54) (end 7.2503 42.54) (width 0.4) (layer B.Cu) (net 21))
 (segment (start 48.7831 43.09) (end 46.9585 41.2654) (width 0.4) (layer F.Cu) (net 21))
 (segment (start 46.9585 41.2654) (end 28.1042 41.2654) (width 0.4) (layer F.Cu) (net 21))
 (segment (start 28.1042 41.2654) (end 8.5249 41.2654) (width 0.4) (layer B.Cu) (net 21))
 (segment (start 8.5249 41.2654) (end 7.2503 42.54) (width 0.4) (layer B.Cu) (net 21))
 (via (at 28.1042 41.2654) (size 0.8) (layers F.Cu B.Cu) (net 21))
 (segment (start 51.7837 62.14) (end 53.7184 62.14) (width 2) (layer B.Cu) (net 11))
 (segment (start 53.7184 62.14) (end 60.0689 55.7895) (width 2) (layer B.Cu) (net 11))
 (segment (start 48.0834 62.14) (end 51.7837 62.14) (width 2) (layer B.Cu) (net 11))
 (via (at 60.0689 55.7895) (size 1) (layers F.Cu B.Cu) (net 11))
 (segment (start 80 5) (end 81.7098 3.2902) (width 1) (layer F.Cu) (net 3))
 (segment (start 81.7098 3.2902) (end 103.5791 3.2902) (width 1) (layer F.Cu) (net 3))
 (segment (start 103.5791 3.2902) (end 135 34.7111) (width 1) (layer F.Cu) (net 3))
 (segment (start 135 34.7111) (end 135 81) (width 1) (layer F.Cu) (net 3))
 (segment (start 6 45.08) (end 7.2503 45.08) (width 0.4) (layer F.Cu) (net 20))
 (segment (start 51.6834 35.47) (end 48.7831 35.47) (width 0.4) (layer F.Cu) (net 20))
 (segment (start 48.7831 35.47) (end 47.3827 34.0696) (width 0.4) (layer F.Cu) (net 20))
 (segment (start 47.3827 34.0696) (end 17.5595 34.0696) (width 0.4) (layer F.Cu) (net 20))
 (segment (start 17.5595 34.0696) (end 7.2503 44.3788) (width 0.4) (layer F.Cu) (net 20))
 (segment (start 7.2503 44.3788) (end 7.2503 45.08) (width 0.4) (layer F.Cu) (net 20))
 (segment (start 78.0834 77.38) (end 74.3831 77.38) (width 2) (layer B.Cu) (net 5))
 (segment (start 74.3831 77.38) (end 74.3831 11.9231) (width 2) (layer B.Cu) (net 5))
 (segment (start 74.3831 11.9231) (end 70 7.54) (width 2) (layer B.Cu) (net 5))
 (segment (start 78.0834 85) (end 82.5022 85) (width 2) (layer B.Cu) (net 2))
 (segment (start 82.5022 85) (end 135 32.5022) (width 2) (layer B.Cu) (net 2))
 (segment (start 135 32.5022) (end 135 27) (width 2) (layer B.Cu) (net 2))
 (segment (start 6 47.62) (end 3.9497 47.62) (width 2) (layer F.Cu) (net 19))
 (segment (start 48.0834 31.66) (end 44.3831 31.66) (width 2) (layer F.Cu) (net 19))
 (segment (start 44.3831 31.66) (end 38.3408 25.6177) (width 2) (layer F.Cu) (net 19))
 (segment (start 38.3408 25.6177) (end 16.9498 25.6177) (width 2) (layer F.Cu) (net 19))
 (segment (start 16.9498 25.6177) (end 3.9497 38.6178) (width 2) (layer F.Cu) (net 19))
 (segment (start 3.9497 38.6178) (end 3.9497 47.62) (width 2) (layer F.Cu) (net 19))
 (segment (start 55.3837 50.71) (end 55.3837 34.5571) (width 2) (layer F.Cu) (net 19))
 (segment (start 55.3837 34.5571) (end 52.4866 31.66) (width 2) (layer F.Cu) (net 19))
 (segment (start 52.4866 31.66) (end 48.0834 31.66) (width 2) (layer F.Cu) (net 19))
 (segment (start 51.6834 50.71) (end 55.3837 50.71) (width 2) (layer F.Cu) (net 19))
 (segment (start 100.32 15.5384) (end 100.32 5) (width 2) (layer F.Cu) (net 11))
 (segment (start 60.0689 55.7895) (end 100.32 15.5384) (width 2) (layer F.Cu) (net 11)))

